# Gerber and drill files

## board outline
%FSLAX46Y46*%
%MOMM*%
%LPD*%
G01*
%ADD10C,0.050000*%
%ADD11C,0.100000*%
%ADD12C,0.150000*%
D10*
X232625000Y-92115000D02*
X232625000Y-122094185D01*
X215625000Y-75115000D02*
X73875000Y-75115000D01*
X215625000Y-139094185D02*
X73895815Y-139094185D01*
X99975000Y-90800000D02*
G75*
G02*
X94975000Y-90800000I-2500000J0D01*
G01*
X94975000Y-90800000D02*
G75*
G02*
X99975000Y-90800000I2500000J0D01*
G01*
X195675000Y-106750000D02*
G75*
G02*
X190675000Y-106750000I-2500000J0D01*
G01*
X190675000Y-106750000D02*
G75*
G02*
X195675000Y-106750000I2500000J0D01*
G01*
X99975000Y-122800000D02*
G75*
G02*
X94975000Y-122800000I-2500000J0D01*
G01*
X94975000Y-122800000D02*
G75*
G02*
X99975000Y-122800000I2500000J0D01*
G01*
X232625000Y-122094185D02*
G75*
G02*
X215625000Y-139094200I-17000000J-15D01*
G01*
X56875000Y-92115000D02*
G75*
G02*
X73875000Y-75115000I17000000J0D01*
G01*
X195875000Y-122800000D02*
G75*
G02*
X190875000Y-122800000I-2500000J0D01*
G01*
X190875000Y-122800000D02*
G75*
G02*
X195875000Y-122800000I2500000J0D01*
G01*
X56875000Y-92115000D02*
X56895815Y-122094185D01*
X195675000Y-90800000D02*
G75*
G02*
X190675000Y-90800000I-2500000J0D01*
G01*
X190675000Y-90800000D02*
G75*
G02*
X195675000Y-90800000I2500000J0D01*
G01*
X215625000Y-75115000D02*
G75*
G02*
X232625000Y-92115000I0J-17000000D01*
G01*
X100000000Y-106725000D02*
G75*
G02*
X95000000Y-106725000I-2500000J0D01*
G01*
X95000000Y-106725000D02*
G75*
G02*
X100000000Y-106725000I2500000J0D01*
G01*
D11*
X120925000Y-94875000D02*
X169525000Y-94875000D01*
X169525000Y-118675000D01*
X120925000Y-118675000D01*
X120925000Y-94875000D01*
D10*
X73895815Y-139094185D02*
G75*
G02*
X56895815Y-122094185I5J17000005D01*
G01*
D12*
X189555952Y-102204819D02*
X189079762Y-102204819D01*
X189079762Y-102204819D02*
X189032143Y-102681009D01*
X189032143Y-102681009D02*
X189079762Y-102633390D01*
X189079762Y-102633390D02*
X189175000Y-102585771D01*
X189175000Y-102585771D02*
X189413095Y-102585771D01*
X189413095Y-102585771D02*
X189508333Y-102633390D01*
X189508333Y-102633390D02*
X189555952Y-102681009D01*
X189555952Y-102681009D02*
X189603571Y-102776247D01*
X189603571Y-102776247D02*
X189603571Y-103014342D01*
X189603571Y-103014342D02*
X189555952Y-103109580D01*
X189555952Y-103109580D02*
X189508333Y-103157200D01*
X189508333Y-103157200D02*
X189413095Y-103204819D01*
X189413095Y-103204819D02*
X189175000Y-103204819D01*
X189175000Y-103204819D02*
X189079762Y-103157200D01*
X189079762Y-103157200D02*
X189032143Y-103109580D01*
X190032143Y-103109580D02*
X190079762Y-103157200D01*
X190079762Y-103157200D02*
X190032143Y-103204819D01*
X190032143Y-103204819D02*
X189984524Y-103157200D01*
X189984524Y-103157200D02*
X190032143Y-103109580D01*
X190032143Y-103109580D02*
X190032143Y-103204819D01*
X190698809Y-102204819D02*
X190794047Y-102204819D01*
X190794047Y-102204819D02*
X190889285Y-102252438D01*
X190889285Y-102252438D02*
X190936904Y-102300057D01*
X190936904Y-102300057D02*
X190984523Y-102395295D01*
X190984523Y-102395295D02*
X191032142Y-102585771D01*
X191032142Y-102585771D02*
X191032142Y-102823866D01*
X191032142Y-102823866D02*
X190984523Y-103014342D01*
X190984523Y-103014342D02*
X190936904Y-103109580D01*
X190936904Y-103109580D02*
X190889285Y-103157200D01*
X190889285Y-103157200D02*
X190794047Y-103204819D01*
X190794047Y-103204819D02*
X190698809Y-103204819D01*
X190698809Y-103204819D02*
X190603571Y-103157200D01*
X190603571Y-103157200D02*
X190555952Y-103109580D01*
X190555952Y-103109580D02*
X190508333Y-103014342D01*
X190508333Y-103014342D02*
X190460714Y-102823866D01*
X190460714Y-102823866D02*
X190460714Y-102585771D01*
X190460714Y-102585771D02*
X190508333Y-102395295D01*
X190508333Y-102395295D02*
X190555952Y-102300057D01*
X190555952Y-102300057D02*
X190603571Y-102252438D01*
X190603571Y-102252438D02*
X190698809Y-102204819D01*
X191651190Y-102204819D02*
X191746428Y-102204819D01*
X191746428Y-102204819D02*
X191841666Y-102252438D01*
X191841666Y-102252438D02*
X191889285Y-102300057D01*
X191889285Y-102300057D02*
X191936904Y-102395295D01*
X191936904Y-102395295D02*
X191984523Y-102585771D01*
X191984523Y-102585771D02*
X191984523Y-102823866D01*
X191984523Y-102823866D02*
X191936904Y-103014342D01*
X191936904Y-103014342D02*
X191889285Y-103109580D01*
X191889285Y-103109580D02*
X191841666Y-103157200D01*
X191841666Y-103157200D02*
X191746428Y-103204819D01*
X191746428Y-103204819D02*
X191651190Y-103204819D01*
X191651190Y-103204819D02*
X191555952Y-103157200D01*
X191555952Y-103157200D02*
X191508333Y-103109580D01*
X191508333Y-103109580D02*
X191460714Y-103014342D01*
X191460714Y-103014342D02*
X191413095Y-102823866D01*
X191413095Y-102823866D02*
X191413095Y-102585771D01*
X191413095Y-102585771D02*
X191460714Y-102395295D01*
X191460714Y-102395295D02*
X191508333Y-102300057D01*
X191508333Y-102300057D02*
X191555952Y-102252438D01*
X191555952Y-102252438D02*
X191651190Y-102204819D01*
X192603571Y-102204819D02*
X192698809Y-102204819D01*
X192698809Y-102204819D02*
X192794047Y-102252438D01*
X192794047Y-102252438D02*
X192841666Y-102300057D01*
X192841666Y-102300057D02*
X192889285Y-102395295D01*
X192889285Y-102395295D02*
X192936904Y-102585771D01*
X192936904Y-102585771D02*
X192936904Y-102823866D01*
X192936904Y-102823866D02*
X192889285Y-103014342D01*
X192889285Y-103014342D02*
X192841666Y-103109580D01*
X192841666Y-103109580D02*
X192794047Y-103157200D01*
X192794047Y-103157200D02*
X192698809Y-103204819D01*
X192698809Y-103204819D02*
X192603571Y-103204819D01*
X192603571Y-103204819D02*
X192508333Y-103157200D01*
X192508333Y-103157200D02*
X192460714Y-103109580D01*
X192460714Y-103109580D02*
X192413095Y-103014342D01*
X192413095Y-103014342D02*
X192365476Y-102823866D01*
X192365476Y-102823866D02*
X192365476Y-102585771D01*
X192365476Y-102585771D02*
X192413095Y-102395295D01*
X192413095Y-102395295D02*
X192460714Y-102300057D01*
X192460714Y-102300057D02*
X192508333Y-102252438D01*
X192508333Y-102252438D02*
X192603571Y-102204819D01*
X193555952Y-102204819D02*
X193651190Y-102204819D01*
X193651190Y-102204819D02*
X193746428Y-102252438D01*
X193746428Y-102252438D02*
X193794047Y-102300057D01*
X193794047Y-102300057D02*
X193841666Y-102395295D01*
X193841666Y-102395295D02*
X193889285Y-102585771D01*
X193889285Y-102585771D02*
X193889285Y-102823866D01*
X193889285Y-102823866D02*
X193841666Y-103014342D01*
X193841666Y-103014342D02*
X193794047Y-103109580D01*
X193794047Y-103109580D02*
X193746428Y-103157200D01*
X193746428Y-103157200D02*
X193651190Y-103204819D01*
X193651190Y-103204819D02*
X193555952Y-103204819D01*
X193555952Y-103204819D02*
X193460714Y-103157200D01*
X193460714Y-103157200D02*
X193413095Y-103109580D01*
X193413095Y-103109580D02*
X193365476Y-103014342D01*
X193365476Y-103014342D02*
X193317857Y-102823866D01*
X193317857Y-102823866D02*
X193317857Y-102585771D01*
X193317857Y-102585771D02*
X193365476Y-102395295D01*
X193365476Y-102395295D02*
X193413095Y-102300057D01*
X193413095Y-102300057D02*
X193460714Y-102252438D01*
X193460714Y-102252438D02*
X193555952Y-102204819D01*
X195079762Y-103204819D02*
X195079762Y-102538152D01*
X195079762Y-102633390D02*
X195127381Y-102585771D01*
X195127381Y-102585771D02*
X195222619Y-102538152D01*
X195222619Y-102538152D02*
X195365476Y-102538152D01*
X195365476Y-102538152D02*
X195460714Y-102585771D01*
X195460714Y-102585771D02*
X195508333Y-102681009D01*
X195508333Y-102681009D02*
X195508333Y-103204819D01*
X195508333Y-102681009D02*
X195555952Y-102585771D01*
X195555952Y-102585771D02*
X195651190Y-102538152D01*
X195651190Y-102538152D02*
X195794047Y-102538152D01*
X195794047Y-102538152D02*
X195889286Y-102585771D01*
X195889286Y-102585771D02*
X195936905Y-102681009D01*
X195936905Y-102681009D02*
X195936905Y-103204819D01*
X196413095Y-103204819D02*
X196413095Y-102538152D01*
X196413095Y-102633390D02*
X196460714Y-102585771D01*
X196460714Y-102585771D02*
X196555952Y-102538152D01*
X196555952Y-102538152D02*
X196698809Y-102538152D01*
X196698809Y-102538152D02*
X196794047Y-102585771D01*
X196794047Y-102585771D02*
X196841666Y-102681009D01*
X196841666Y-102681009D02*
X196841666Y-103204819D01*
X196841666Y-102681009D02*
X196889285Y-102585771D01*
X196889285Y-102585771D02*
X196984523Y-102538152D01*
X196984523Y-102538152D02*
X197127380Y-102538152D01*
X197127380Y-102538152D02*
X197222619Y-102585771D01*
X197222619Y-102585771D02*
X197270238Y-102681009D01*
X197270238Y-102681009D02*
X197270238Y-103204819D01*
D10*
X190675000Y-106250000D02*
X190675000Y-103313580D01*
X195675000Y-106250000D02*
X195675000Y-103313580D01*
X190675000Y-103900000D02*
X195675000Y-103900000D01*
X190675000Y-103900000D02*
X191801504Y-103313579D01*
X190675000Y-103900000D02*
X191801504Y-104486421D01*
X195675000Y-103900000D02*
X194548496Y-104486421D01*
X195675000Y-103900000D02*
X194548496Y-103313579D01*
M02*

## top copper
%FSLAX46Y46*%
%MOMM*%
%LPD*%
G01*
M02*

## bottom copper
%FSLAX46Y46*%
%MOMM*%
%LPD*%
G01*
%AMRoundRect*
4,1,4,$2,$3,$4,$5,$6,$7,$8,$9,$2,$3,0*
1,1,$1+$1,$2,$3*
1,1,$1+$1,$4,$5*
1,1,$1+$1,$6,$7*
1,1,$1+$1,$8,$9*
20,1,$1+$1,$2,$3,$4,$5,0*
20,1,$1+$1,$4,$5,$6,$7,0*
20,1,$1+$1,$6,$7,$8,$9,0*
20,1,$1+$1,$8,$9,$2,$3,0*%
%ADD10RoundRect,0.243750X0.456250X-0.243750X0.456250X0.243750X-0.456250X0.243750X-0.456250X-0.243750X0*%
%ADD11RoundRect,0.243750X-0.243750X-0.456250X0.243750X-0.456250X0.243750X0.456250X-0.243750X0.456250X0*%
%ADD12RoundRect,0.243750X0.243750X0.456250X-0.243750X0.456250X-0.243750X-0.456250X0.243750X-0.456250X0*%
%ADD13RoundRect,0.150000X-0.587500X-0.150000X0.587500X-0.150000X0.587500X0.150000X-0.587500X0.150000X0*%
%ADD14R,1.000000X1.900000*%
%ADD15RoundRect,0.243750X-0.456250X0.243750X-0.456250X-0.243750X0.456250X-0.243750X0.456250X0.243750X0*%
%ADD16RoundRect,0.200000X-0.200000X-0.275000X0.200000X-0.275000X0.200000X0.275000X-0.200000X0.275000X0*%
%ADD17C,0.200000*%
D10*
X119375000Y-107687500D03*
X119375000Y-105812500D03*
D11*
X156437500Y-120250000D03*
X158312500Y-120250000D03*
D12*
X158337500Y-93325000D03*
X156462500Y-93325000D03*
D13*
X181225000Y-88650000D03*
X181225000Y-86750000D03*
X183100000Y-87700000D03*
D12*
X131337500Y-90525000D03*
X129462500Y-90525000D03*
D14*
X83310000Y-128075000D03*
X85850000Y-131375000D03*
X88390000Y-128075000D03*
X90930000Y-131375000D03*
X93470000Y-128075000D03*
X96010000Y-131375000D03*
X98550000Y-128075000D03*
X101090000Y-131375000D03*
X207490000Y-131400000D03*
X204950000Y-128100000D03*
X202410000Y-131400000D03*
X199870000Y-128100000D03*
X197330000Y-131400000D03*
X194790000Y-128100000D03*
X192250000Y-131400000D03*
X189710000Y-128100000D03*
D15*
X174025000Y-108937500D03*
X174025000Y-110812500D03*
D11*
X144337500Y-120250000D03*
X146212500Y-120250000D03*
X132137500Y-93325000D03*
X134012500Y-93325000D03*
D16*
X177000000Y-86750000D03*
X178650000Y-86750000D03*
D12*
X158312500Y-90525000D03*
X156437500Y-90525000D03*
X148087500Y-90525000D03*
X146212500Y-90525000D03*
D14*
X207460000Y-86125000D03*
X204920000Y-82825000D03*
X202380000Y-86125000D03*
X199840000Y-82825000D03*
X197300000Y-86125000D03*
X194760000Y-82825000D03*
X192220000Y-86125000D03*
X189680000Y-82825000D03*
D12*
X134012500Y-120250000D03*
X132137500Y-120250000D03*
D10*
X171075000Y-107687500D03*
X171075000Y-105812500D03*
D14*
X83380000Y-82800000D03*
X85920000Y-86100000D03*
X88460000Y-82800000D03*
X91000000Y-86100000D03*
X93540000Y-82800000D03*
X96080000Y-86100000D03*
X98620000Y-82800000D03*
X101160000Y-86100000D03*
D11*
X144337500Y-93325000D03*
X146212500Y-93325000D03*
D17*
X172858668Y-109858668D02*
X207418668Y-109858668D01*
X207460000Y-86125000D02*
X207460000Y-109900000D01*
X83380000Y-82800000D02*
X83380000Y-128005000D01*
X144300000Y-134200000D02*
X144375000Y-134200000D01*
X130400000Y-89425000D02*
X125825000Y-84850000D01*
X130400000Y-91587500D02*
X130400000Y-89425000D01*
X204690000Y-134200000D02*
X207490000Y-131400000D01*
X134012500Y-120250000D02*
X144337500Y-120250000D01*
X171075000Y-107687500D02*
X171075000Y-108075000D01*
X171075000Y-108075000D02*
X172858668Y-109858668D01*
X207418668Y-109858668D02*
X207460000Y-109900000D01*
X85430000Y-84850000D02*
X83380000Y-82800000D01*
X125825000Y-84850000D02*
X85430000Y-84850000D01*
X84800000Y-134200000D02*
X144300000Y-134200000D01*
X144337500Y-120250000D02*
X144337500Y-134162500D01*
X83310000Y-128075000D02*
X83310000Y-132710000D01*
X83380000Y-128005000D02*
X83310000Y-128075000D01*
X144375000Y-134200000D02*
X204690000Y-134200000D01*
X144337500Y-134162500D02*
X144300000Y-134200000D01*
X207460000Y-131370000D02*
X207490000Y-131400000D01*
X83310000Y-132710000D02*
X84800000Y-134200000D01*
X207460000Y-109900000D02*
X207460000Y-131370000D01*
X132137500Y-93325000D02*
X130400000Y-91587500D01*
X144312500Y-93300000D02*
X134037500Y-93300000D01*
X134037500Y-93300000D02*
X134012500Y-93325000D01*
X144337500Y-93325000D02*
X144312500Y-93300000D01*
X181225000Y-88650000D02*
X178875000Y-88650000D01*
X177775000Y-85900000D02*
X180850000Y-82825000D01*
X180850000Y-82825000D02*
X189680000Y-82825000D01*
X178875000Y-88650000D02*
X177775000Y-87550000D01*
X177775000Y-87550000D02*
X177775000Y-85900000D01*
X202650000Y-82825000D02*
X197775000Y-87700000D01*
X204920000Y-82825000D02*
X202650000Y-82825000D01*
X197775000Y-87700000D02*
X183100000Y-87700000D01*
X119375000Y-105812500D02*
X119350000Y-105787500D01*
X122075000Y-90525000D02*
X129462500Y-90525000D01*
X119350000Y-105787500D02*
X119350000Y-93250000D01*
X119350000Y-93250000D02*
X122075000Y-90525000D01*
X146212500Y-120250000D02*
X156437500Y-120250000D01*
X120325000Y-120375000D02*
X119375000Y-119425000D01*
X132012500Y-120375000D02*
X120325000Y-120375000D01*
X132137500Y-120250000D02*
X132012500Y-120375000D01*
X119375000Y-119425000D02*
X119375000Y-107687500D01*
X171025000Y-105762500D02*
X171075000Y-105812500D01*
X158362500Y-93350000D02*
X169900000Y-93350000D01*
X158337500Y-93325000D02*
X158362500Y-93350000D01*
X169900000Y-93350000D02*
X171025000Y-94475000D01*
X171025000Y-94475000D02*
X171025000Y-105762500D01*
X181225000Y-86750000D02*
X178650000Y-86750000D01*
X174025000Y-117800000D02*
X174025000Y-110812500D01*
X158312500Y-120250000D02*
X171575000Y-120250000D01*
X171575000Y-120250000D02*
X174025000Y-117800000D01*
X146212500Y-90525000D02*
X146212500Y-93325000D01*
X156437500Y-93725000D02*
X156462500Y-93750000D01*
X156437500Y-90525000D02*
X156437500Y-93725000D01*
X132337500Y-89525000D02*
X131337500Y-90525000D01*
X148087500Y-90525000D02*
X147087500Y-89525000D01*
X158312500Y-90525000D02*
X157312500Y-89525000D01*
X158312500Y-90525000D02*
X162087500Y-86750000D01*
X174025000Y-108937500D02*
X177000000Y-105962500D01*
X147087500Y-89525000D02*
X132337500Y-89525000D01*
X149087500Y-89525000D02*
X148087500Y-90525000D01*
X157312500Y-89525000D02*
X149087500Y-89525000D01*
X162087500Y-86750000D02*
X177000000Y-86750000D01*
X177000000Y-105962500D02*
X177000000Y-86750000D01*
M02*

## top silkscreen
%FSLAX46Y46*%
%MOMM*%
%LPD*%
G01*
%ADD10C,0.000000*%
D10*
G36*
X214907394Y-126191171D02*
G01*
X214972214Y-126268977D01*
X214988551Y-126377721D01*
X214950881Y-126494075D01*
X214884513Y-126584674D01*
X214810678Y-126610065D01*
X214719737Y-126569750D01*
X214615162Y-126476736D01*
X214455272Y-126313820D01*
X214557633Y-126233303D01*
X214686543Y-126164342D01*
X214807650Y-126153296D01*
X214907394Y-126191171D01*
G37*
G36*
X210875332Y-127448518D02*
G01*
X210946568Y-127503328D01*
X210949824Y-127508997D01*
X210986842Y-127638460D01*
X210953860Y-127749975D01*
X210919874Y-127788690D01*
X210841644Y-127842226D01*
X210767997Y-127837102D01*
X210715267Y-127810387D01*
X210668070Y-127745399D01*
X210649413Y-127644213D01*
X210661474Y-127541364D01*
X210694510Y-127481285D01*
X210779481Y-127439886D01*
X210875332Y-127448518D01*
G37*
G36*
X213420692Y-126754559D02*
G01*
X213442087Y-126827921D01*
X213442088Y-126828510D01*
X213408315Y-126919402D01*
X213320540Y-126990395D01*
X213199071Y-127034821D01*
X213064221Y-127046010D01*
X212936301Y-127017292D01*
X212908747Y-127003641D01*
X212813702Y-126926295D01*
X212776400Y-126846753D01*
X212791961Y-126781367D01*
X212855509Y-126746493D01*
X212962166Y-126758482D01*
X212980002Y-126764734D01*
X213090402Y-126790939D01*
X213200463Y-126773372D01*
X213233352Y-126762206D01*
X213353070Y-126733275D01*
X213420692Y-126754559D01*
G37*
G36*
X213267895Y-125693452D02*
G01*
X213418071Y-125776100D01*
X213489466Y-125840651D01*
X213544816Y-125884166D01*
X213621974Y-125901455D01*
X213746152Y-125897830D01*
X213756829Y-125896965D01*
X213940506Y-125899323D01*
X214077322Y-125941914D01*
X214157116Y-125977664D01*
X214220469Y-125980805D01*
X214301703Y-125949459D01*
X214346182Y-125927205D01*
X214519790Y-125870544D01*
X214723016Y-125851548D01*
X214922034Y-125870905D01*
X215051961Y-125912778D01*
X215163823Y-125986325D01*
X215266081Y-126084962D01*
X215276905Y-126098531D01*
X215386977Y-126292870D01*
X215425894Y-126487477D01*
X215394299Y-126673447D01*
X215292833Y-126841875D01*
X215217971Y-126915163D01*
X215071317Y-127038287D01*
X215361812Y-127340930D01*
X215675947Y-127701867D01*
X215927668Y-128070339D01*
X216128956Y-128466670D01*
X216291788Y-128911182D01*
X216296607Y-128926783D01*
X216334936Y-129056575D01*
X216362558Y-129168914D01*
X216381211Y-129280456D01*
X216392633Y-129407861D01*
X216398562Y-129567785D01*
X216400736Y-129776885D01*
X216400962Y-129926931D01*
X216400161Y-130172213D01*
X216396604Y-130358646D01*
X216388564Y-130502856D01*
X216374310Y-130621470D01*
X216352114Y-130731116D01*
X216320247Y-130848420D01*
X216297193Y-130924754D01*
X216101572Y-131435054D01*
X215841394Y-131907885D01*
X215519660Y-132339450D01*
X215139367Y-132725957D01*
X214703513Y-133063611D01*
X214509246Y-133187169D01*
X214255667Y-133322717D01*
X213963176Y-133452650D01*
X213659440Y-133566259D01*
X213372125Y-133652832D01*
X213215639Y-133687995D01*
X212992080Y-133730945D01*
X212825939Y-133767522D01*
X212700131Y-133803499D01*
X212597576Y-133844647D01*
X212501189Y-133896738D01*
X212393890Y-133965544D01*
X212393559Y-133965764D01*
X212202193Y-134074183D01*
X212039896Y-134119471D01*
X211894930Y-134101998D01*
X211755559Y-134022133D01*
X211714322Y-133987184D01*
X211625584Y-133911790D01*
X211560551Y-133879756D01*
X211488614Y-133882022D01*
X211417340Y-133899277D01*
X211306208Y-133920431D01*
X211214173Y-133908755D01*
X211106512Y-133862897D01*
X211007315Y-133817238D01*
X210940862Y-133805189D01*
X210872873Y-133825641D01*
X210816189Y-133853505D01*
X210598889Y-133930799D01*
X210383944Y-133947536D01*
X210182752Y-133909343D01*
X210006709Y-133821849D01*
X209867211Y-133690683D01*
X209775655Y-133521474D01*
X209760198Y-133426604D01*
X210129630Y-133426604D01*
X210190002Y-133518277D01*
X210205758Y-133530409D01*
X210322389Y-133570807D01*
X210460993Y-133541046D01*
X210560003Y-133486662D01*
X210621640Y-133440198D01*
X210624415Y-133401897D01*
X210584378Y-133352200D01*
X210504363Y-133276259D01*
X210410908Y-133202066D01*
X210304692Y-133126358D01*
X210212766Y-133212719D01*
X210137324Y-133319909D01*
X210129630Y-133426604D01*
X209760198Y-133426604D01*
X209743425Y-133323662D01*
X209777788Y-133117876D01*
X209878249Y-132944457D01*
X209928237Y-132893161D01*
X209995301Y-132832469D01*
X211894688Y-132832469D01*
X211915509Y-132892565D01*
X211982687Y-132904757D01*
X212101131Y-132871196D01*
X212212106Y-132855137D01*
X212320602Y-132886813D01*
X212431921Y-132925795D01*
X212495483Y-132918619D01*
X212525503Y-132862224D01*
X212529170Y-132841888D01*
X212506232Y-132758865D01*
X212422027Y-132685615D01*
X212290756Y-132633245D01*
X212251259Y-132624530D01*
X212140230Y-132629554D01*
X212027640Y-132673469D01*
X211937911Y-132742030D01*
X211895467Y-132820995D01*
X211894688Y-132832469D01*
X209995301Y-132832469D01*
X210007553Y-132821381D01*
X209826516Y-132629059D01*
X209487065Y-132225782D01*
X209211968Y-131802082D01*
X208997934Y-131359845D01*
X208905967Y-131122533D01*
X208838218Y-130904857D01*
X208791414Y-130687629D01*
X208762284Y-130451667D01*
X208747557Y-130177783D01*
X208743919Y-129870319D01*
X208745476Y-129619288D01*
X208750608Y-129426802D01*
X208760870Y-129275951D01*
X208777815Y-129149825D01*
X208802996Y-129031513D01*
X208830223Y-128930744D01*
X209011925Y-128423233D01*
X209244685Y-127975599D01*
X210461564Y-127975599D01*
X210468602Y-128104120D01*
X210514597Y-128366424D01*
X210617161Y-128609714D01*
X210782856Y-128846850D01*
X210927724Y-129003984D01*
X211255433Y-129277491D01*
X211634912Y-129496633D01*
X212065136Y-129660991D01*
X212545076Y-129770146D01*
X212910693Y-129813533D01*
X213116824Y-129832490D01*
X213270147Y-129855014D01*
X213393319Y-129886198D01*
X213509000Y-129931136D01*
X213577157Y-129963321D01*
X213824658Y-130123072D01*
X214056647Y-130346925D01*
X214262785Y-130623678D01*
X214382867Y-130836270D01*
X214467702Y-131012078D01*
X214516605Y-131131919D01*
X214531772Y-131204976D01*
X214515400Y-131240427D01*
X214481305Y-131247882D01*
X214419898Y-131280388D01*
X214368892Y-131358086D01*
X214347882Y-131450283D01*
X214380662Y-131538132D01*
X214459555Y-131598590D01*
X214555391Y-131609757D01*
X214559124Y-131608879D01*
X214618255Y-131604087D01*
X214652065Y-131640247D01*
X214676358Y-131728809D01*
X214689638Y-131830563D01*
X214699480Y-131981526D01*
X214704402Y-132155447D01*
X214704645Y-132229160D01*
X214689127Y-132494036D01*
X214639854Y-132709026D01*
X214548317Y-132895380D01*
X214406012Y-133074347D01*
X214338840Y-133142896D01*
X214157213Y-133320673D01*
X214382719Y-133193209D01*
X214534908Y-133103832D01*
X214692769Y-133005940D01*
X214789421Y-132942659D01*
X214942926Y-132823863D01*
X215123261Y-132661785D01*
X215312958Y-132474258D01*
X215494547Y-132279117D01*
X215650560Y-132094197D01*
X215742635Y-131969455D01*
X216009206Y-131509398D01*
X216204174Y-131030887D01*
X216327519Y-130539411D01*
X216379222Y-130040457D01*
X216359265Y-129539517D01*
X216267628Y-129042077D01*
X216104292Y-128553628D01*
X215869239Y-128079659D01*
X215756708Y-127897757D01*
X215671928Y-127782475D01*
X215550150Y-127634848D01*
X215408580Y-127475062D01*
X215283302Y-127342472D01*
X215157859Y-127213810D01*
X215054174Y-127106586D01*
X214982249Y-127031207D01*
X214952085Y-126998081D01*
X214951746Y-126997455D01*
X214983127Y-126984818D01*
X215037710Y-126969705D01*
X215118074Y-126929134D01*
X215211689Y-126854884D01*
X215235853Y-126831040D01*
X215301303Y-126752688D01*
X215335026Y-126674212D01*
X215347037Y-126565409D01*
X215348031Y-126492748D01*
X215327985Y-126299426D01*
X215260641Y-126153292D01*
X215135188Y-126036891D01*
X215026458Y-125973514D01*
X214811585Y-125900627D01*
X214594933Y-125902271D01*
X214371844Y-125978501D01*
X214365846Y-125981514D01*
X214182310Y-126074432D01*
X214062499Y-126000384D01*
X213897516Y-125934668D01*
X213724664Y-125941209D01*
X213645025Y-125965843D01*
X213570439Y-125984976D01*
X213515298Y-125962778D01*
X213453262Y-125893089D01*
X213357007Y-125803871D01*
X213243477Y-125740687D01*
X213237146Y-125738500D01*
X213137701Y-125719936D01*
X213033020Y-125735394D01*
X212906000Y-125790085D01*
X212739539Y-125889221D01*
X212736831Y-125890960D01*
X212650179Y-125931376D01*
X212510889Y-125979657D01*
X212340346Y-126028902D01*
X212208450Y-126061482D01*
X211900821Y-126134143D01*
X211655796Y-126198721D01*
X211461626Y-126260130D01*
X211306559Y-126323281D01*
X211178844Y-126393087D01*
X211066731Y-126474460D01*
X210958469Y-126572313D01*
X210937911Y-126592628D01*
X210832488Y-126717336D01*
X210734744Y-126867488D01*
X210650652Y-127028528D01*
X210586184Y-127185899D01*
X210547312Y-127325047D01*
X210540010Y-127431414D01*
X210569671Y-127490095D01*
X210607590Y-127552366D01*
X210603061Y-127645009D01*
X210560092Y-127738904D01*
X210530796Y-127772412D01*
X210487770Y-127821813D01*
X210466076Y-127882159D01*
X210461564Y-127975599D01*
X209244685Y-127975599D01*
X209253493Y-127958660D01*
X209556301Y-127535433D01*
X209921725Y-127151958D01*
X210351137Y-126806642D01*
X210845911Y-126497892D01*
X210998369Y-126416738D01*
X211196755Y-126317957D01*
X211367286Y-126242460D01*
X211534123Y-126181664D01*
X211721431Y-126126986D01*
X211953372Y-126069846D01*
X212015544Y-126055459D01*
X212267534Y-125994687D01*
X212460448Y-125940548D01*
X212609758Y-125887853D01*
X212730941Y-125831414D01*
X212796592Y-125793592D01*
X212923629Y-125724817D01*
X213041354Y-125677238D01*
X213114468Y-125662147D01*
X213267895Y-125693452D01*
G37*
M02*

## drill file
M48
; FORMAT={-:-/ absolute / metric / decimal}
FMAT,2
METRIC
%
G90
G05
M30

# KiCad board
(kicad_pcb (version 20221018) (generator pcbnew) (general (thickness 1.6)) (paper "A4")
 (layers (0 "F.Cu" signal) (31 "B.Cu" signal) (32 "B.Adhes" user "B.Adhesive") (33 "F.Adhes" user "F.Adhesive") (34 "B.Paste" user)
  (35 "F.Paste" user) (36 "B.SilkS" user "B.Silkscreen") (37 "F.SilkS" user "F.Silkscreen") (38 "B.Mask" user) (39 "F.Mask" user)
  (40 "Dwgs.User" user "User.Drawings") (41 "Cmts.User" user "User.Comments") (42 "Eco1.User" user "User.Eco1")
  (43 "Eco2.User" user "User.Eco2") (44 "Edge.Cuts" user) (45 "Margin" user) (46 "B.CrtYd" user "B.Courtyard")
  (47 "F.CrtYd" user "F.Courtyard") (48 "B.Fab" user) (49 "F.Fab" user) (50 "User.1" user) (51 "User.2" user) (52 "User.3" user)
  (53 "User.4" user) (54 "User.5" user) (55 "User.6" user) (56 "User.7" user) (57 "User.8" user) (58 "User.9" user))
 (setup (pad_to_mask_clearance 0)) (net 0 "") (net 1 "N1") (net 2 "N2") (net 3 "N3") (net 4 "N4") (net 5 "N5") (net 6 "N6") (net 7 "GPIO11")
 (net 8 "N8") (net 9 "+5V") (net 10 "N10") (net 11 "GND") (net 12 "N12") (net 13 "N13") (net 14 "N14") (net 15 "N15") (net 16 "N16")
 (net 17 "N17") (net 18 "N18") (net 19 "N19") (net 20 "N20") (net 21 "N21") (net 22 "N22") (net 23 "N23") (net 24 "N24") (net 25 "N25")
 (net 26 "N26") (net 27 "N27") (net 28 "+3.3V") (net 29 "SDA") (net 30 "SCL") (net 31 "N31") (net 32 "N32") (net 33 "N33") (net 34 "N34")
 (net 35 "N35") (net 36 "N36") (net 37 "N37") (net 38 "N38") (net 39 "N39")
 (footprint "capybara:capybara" (layer "F.Cu") (at 212.725 129.625)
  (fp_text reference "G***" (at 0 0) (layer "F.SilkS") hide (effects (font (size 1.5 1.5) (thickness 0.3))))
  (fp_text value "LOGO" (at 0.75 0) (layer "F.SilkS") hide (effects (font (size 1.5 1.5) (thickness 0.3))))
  (fp_poly
   (pts (xy 2.182394 -3.433829) (xy 2.247214 -3.356023) (xy 2.263551 -3.247279) (xy 2.225881 -3.130925) (xy 2.159513 -3.040326)
    (xy 2.085678 -3.014935) (xy 1.994737 -3.05525) (xy 1.890162 -3.148264) (xy 1.730272 -3.31118) (xy 1.832633 -3.391697)
    (xy 1.961543 -3.460658) (xy 2.08265 -3.471704))
   (stroke (width 0) (type solid)) (fill solid) (layer "F.SilkS"))
  (fp_poly
   (pts (xy -1.849668 -2.176482) (xy -1.778432 -2.121672) (xy -1.775176 -2.116003) (xy -1.738158 -1.98654) (xy -1.77114 -1.875025)
    (xy -1.805126 -1.83631) (xy -1.883356 -1.782774) (xy -1.957003 -1.787898) (xy -2.009733 -1.814613) (xy -2.05693 -1.879601)
    (xy -2.075587 -1.980787) (xy -2.063526 -2.083636) (xy -2.03049 -2.143715) (xy -1.945519 -2.185114))
   (stroke (width 0) (type solid)) (fill solid) (layer "F.SilkS"))
  (fp_poly
   (pts (xy 0.695692 -2.870441) (xy 0.717087 -2.797079) (xy 0.717088 -2.79649) (xy 0.683315 -2.705598) (xy 0.59554 -2.634605)
    (xy 0.474071 -2.590179) (xy 0.339221 -2.57899) (xy 0.211301 -2.607708) (xy 0.183747 -2.621359) (xy 0.088702 -2.698705)
    (xy 0.0514 -2.778247) (xy 0.066961 -2.843633) (xy 0.130509 -2.878507) (xy 0.237166 -2.866518) (xy 0.255002 -2.860266)
    (xy 0.365402 -2.834061) (xy 0.475463 -2.851628) (xy 0.508352 -2.862794) (xy 0.62807 -2.891725))
   (stroke (width 0) (type solid)) (fill solid) (layer "F.SilkS"))
  (fp_poly
   (pts (xy 0.542895 -3.931548) (xy 0.693071 -3.8489) (xy 0.764466 -3.784349) (xy 0.819816 -3.740834) (xy 0.896974 -3.723545)
    (xy 1.021152 -3.72717) (xy 1.031829 -3.728035) (xy 1.215506 -3.725677) (xy 1.352322 -3.683086) (xy 1.432116 -3.647336)
    (xy 1.495469 -3.644195) (xy 1.576703 -3.675541) (xy 1.621182 -3.697795) (xy 1.79479 -3.754456) (xy 1.998016 -3.773452)
    (xy 2.197034 -3.754095) (xy 2.326961 -3.712222) (xy 2.438823 -3.638675) (xy 2.541081 -3.540038) (xy 2.551905 -3.526469)
    (xy 2.661977 -3.33213) (xy 2.700894 -3.137523) (xy 2.669299 -2.951553) (xy 2.567833 -2.783125) (xy 2.492971 -2.709837)
    (xy 2.346317 -2.586713) (xy 2.636812 -2.28407) (xy 2.950947 -1.923133) (xy 3.202668 -1.554661) (xy 3.403956 -1.15833)
    (xy 3.566788 -0.713818) (xy 3.571607 -0.698217) (xy 3.609936 -0.568425) (xy 3.637558 -0.456086) (xy 3.656211 -0.344544)
    (xy 3.667633 -0.217139) (xy 3.673562 -0.057215) (xy 3.675736 0.151885) (xy 3.675962 0.301931) (xy 3.675161 0.547213)
    (xy 3.671604 0.733646) (xy 3.663564 0.877856) (xy 3.64931 0.99647) (xy 3.627114 1.106116) (xy 3.595247 1.22342) (xy 3.572193 1.299754)
    (xy 3.376572 1.810054) (xy 3.116394 2.282885) (xy 2.79466 2.71445) (xy 2.414367 3.100957) (xy 1.978513 3.438611) (xy 1.784246 3.562169)
    (xy 1.530667 3.697717) (xy 1.238176 3.82765) (xy 0.93444 3.941259) (xy 0.647125 4.027832) (xy 0.490639 4.062995) (xy 0.26708 4.105945)
    (xy 0.100939 4.142522) (xy -0.024869 4.178499) (xy -0.127424 4.219647) (xy -0.223811 4.271738) (xy -0.33111 4.340544)
    (xy -0.331441 4.340764) (xy -0.522807 4.449183) (xy -0.685104 4.494471) (xy -0.83007 4.476998) (xy -0.969441 4.397133)
    (xy -1.010678 4.362184) (xy -1.099416 4.28679) (xy -1.164449 4.254756) (xy -1.236386 4.257022) (xy -1.30766 4.274277)
    (xy -1.418792 4.295431) (xy -1.510827 4.283755) (xy -1.618488 4.237897) (xy -1.717685 4.192238) (xy -1.784138 4.180189)
    (xy -1.852127 4.200641) (xy -1.908811 4.228505) (xy -2.126111 4.305799) (xy -2.341056 4.322536) (xy -2.542248 4.284343)
    (xy -2.718291 4.196849) (xy -2.857789 4.065683) (xy -2.949345 3.896474) (xy -2.964802 3.801604) (xy -2.59537 3.801604)
    (xy -2.534998 3.893277) (xy -2.519242 3.905409) (xy -2.402611 3.945807) (xy -2.264007 3.916046) (xy -2.164997 3.861662)
    (xy -2.10336 3.815198) (xy -2.100585 3.776897) (xy -2.140622 3.7272) (xy -2.220637 3.651259) (xy -2.314092 3.577066)
    (xy -2.420308 3.501358) (xy -2.512234 3.587719) (xy -2.587676 3.694909) (xy -2.59537 3.801604) (xy -2.964802 3.801604)
    (xy -2.981575 3.698662) (xy -2.947212 3.492876) (xy -2.846751 3.319457) (xy -2.796763 3.268161) (xy -2.729699 3.207469)
    (xy -0.830312 3.207469) (xy -0.809491 3.267565) (xy -0.742313 3.279757) (xy -0.623869 3.246196) (xy -0.512894 3.230137)
    (xy -0.404398 3.261813) (xy -0.293079 3.300795) (xy -0.229517 3.293619) (xy -0.199497 3.237224) (xy -0.19583 3.216888)
    (xy -0.218768 3.133865) (xy -0.302973 3.060615) (xy -0.434244 3.008245) (xy -0.473741 2.99953) (xy -0.58477 3.004554)
    (xy -0.69736 3.048469) (xy -0.787089 3.11703) (xy -0.829533 3.195995) (xy -0.830312 3.207469) (xy -2.729699 3.207469)
    (xy -2.717447 3.196381) (xy -2.898484 3.004059) (xy -3.237935 2.600782) (xy -3.513032 2.177082) (xy -3.727066 1.734845)
    (xy -3.819033 1.497533) (xy -3.886782 1.279857) (xy -3.933586 1.062629) (xy -3.962716 0.826667) (xy -3.977443 0.552783)
    (xy -3.981081 0.245319) (xy -3.979524 -0.005712) (xy -3.974392 -0.198198) (xy -3.96413 -0.349049) (xy -3.947185 -0.475175)
    (xy -3.922004 -0.593487) (xy -3.894777 -0.694256) (xy -3.713075 -1.201767) (xy -3.480315 -1.649401) (xy -2.263436 -1.649401)
    (xy -2.256398 -1.52088) (xy -2.210403 -1.258576) (xy -2.107839 -1.015286) (xy -1.942144 -0.77815) (xy -1.797276 -0.621016)
    (xy -1.469567 -0.347509) (xy -1.090088 -0.128367) (xy -0.659864 0.035991) (xy -0.179924 0.145146) (xy 0.185693 0.188533)
    (xy 0.391824 0.20749) (xy 0.545147 0.230014) (xy 0.668319 0.261198) (xy 0.784 0.306136) (xy 0.852157 0.338321) (xy 1.099658 0.498072)
    (xy 1.331647 0.721925) (xy 1.537785 0.998678) (xy 1.657867 1.21127) (xy 1.742702 1.387078) (xy 1.791605 1.506919) (xy 1.806772 1.579976)
    (xy 1.7904 1.615427) (xy 1.756305 1.622882) (xy 1.694898 1.655388) (xy 1.643892 1.733086) (xy 1.622882 1.825283) (xy 1.655662 1.913132)
    (xy 1.734555 1.97359) (xy 1.830391 1.984757) (xy 1.834124 1.983879) (xy 1.893255 1.979087) (xy 1.927065 2.015247) (xy 1.951358 2.103809)
    (xy 1.964638 2.205563) (xy 1.97448 2.356526) (xy 1.979402 2.530447) (xy 1.979645 2.60416) (xy 1.964127 2.869036) (xy 1.914854 3.084026)
    (xy 1.823317 3.27038) (xy 1.681012 3.449347) (xy 1.61384 3.517896) (xy 1.432213 3.695673) (xy 1.657719 3.568209) (xy 1.809908 3.478832)
    (xy 1.967769 3.38094) (xy 2.064421 3.317659) (xy 2.217926 3.198863) (xy 2.398261 3.036785) (xy 2.587958 2.849258) (xy 2.769547 2.654117)
    (xy 2.92556 2.469197) (xy 3.017635 2.344455) (xy 3.284206 1.884398) (xy 3.479174 1.405887) (xy 3.602519 0.914411) (xy 3.654222 0.415457)
    (xy 3.634265 -0.085483) (xy 3.542628 -0.582923) (xy 3.379292 -1.071372) (xy 3.144239 -1.545341) (xy 3.031708 -1.727243)
    (xy 2.946928 -1.842525) (xy 2.82515 -1.990152) (xy 2.68358 -2.149938) (xy 2.558302 -2.282528) (xy 2.432859 -2.41119)
    (xy 2.329174 -2.518414) (xy 2.257249 -2.593793) (xy 2.227085 -2.626919) (xy 2.226746 -2.627545) (xy 2.258127 -2.640182)
    (xy 2.31271 -2.655295) (xy 2.393074 -2.695866) (xy 2.486689 -2.770116) (xy 2.510853 -2.79396) (xy 2.576303 -2.872312)
    (xy 2.610026 -2.950788) (xy 2.622037 -3.059591) (xy 2.623031 -3.132252) (xy 2.602985 -3.325574) (xy 2.535641 -3.471708)
    (xy 2.410188 -3.588109) (xy 2.301458 -3.651486) (xy 2.086585 -3.724373) (xy 1.869933 -3.722729) (xy 1.646844 -3.646499)
    (xy 1.640846 -3.643486) (xy 1.45731 -3.550568) (xy 1.337499 -3.624616) (xy 1.172516 -3.690332) (xy 0.999664 -3.683791)
    (xy 0.920025 -3.659157) (xy 0.845439 -3.640024) (xy 0.790298 -3.662222) (xy 0.728262 -3.731911) (xy 0.632007 -3.821129)
    (xy 0.518477 -3.884313) (xy 0.512146 -3.8865) (xy 0.412701 -3.905064) (xy 0.30802 -3.889606) (xy 0.181 -3.834915)
    (xy 0.014539 -3.735779) (xy 0.011831 -3.73404) (xy -0.074821 -3.693624) (xy -0.214111 -3.645343) (xy -0.384654 -3.596098)
    (xy -0.51655 -3.563518) (xy -0.824179 -3.490857) (xy -1.069204 -3.426279) (xy -1.263374 -3.36487) (xy -1.418441 -3.301719)
    (xy -1.546156 -3.231913) (xy -1.658269 -3.15054) (xy -1.766531 -3.052687) (xy -1.787089 -3.032372) (xy -1.892512 -2.907664)
    (xy -1.990256 -2.757512) (xy -2.074348 -2.596472) (xy -2.138816 -2.439101) (xy -2.177688 -2.299953) (xy -2.18499 -2.193586)
    (xy -2.155329 -2.134905) (xy -2.11741 -2.072634) (xy -2.121939 -1.979991) (xy -2.164908 -1.886096) (xy -2.194204 -1.852588)
    (xy -2.23723 -1.803187) (xy -2.258924 -1.742841) (xy -2.263436 -1.649401) (xy -3.480315 -1.649401) (xy -3.471507 -1.66634)
    (xy -3.168699 -2.089567) (xy -2.803275 -2.473042) (xy -2.373863 -2.818358) (xy -1.879089 -3.127108) (xy -1.726631 -3.208262)
    (xy -1.528245 -3.307043) (xy -1.357714 -3.38254) (xy -1.190877 -3.443336) (xy -1.003569 -3.498014) (xy -0.771628 -3.555154)
    (xy -0.709456 -3.569541) (xy -0.457466 -3.630313) (xy -0.264552 -3.684452) (xy -0.115242 -3.737147) (xy 0.005941 -3.793586)
    (xy 0.071592 -3.831408) (xy 0.198629 -3.900183) (xy 0.316354 -3.947762) (xy 0.389468 -3.962853))
   (stroke (width 0) (type solid)) (fill solid) (layer "F.SilkS")))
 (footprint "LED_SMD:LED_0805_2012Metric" (layer "B.Cu") (at 119.375 106.75 90)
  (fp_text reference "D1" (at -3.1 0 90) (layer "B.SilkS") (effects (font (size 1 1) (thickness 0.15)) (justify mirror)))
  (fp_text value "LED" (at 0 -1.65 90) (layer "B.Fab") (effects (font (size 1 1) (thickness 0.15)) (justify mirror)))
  (pad "1" smd roundrect (at -0.9375 0 90) (size 0.975 1.4) (layers "B.Cu" "B.Paste" "B.Mask") (roundrect_rratio 0.25) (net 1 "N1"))
  (pad "2" smd roundrect (at 0.9375 0 90) (size 0.975 1.4) (layers "B.Cu" "B.Paste" "B.Mask") (roundrect_rratio 0.25) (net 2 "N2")))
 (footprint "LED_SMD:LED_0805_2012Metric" (layer "B.Cu") (at 157.375 120.25)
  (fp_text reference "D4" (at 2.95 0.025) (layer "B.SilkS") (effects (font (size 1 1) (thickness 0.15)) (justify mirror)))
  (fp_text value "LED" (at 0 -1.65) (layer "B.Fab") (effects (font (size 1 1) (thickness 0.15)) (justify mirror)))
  (pad "1" smd roundrect (at -0.9375 0) (size 0.975 1.4) (layers "B.Cu" "B.Paste" "B.Mask") (roundrect_rratio 0.25) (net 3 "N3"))
  (pad "2" smd roundrect (at 0.9375 0) (size 0.975 1.4) (layers "B.Cu" "B.Paste" "B.Mask") (roundrect_rratio 0.25) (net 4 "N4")))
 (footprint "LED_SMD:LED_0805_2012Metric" (layer "B.Cu") (at 157.4 93.325 180)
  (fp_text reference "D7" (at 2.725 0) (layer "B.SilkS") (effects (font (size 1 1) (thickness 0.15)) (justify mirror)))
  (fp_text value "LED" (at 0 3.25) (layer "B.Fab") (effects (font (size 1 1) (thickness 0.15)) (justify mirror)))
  (pad "1" smd roundrect (at -0.9375 0 180) (size 0.975 1.4) (layers "B.Cu" "B.Paste" "B.Mask") (roundrect_rratio 0.25) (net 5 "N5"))
  (pad "2" smd roundrect (at 0.9375 0 180) (size 0.975 1.4) (layers "B.Cu" "B.Paste" "B.Mask") (roundrect_rratio 0.25) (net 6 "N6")))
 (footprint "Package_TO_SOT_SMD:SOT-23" (layer "B.Cu") (at 182.1625 87.7)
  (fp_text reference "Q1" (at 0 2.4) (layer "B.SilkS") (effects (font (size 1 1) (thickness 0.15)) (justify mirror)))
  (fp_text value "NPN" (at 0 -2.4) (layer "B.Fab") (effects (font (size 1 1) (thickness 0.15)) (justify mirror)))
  (pad "1" smd roundrect (at -0.9375 0.95) (size 1.475 0.6) (layers "B.Cu" "B.Paste" "B.Mask") (roundrect_rratio 0.25) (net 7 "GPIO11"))
  (pad "2" smd roundrect (at -0.9375 -0.95) (size 1.475 0.6) (layers "B.Cu" "B.Paste" "B.Mask") (roundrect_rratio 0.25) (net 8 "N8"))
  (pad "3" smd roundrect (at 0.9375 0) (size 1.475 0.6) (layers "B.Cu" "B.Paste" "B.Mask") (roundrect_rratio 0.25) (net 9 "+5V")))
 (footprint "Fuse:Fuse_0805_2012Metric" (layer "B.Cu") (at 130.4 90.525 180)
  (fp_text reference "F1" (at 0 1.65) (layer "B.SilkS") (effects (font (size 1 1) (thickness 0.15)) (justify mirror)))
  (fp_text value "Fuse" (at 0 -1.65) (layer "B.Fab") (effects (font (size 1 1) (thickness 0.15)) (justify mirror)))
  (pad "1" smd roundrect (at -0.9375 0 180) (size 0.975 1.4) (layers "B.Cu" "B.Paste" "B.Mask") (roundrect_rratio 0.25) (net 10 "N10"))
  (pad "2" smd roundrect (at 0.9375 0 180) (size 0.975 1.4) (layers "B.Cu" "B.Paste" "B.Mask") (roundrect_rratio 0.25) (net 2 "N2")))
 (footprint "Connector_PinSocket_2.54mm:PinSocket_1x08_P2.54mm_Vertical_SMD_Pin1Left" (layer "B.Cu") (at 92.2 129.725 -90)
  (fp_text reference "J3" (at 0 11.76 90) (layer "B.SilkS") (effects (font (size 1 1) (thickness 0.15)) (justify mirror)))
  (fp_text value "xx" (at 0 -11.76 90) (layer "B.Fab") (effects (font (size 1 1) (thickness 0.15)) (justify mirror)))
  (pad "1" smd rect (at -1.65 8.89 270) (size 1.9 1) (layers "B.Cu" "B.Paste" "B.Mask") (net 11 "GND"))
  (pad "2" smd rect (at 1.65 6.35 270) (size 1.9 1) (layers "B.Cu" "B.Paste" "B.Mask") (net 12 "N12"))
  (pad "3" smd rect (at -1.65 3.81 270) (size 1.9 1) (layers "B.Cu" "B.Paste" "B.Mask") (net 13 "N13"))
  (pad "4" smd rect (at 1.65 1.27 270) (size 1.9 1) (layers "B.Cu" "B.Paste" "B.Mask") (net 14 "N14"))
  (pad "5" smd rect (at -1.65 -1.27 270) (size 1.9 1) (layers "B.Cu" "B.Paste" "B.Mask") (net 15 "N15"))
  (pad "6" smd rect (at 1.65 -3.81 270) (size 1.9 1) (layers "B.Cu" "B.Paste" "B.Mask") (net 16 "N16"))
  (pad "7" smd rect (at -1.65 -6.35 270) (size 1.9 1) (layers "B.Cu" "B.Paste" "B.Mask") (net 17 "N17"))
  (pad "8" smd rect (at 1.65 -8.89 270) (size 1.9 1) (layers "B.Cu" "B.Paste" "B.Mask") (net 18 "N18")))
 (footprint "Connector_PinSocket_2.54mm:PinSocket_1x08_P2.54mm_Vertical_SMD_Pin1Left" (layer "B.Cu") (at 198.6 129.75 90)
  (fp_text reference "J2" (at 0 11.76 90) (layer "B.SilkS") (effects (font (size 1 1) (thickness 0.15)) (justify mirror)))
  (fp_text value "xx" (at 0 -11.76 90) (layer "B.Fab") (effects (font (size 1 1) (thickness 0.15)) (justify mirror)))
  (pad "1" smd rect (at -1.65 8.89 90) (size 1.9 1) (layers "B.Cu" "B.Paste" "B.Mask") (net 11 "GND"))
  (pad "2" smd rect (at 1.65 6.35 90) (size 1.9 1) (layers "B.Cu" "B.Paste" "B.Mask") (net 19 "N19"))
  (pad "3" smd rect (at -1.65 3.81 90) (size 1.9 1) (layers "B.Cu" "B.Paste" "B.Mask") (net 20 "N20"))
  (pad "4" smd rect (at 1.65 1.27 90) (size 1.9 1) (layers "B.Cu" "B.Paste" "B.Mask") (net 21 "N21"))
  (pad "5" smd rect (at -1.65 -1.27 90) (size 1.9 1) (layers "B.Cu" "B.Paste" "B.Mask") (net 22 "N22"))
  (pad "6" smd rect (at 1.65 -3.81 90) (size 1.9 1) (layers "B.Cu" "B.Paste" "B.Mask") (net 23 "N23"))
  (pad "7" smd rect (at -1.65 -6.35 90) (size 1.9 1) (layers "B.Cu" "B.Paste" "B.Mask") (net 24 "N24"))
  (pad "8" smd rect (at 1.65 -8.89 90) (size 1.9 1) (layers "B.Cu" "B.Paste" "B.Mask") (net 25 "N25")))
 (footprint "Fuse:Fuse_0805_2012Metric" (layer "B.Cu") (at 174.025 109.875 -90)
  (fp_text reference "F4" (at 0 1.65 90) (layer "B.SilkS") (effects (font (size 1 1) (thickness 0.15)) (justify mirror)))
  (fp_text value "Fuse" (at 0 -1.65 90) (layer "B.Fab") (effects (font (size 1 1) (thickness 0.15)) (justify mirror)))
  (pad "1" smd roundrect (at -0.9375 0 270) (size 0.975 1.4) (layers "B.Cu" "B.Paste" "B.Mask") (roundrect_rratio 0.25) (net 10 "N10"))
  (pad "2" smd roundrect (at 0.9375 0 270) (size 0.975 1.4) (layers "B.Cu" "B.Paste" "B.Mask") (roundrect_rratio 0.25) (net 4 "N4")))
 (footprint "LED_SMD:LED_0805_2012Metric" (layer "B.Cu") (at 145.275 120.25)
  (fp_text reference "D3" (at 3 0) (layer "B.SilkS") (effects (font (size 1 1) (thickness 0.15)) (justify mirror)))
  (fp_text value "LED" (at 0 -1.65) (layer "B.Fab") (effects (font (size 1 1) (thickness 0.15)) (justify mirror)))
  (pad "1" smd roundrect (at -0.9375 0) (size 0.975 1.4) (layers "B.Cu" "B.Paste" "B.Mask") (roundrect_rratio 0.25) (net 11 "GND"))
  (pad "2" smd roundrect (at 0.9375 0) (size 0.975 1.4) (layers "B.Cu" "B.Paste" "B.Mask") (roundrect_rratio 0.25) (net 3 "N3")))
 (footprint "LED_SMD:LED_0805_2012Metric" (layer "B.Cu") (at 133.075 93.325)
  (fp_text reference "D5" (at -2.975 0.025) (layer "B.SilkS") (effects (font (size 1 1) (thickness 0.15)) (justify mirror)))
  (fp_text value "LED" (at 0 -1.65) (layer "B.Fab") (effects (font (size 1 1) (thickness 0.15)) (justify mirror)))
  (pad "1" smd roundrect (at -0.9375 0) (size 0.975 1.4) (layers "B.Cu" "B.Paste" "B.Mask") (roundrect_rratio 0.25) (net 11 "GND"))
  (pad "2" smd roundrect (at 0.9375 0) (size 0.975 1.4) (layers "B.Cu" "B.Paste" "B.Mask") (roundrect_rratio 0.25) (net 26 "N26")))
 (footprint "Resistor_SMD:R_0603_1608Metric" (layer "B.Cu") (at 177.825 86.75)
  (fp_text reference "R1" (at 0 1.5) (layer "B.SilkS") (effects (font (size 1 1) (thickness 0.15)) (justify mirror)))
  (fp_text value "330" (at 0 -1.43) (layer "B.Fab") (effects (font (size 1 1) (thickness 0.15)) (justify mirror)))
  (pad "1" smd roundrect (at -0.825 0) (size 0.8 0.95) (layers "B.Cu" "B.Paste" "B.Mask") (roundrect_rratio 0.25) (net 10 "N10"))
  (pad "2" smd roundrect (at 0.825 0) (size 0.8 0.95) (layers "B.Cu" "B.Paste" "B.Mask") (roundrect_rratio 0.25) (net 8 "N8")))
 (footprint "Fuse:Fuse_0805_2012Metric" (layer "B.Cu") (at 157.375 90.525 180)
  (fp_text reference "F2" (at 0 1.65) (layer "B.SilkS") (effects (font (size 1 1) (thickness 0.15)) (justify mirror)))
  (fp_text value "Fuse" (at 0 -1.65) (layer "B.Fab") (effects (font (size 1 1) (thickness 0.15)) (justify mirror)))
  (pad "1" smd roundrect (at -0.9375 0 180) (size 0.975 1.4) (layers "B.Cu" "B.Paste" "B.Mask") (roundrect_rratio 0.25) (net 10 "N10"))
  (pad "2" smd roundrect (at 0.9375 0 180) (size 0.975 1.4) (layers "B.Cu" "B.Paste" "B.Mask") (roundrect_rratio 0.25) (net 6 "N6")))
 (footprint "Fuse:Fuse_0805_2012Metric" (layer "B.Cu") (at 147.15 90.525 180)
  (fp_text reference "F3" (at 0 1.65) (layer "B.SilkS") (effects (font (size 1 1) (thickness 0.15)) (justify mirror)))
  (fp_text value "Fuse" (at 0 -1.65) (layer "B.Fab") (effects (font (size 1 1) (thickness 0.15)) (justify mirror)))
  (pad "1" smd roundrect (at -0.9375 0 180) (size 0.975 1.4) (layers "B.Cu" "B.Paste" "B.Mask") (roundrect_rratio 0.25) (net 10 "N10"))
  (pad "2" smd roundrect (at 0.9375 0 180) (size 0.975 1.4) (layers "B.Cu" "B.Paste" "B.Mask") (roundrect_rratio 0.25) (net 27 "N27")))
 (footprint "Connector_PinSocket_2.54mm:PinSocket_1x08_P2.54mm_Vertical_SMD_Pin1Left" (layer "B.Cu") (at 198.57 84.475 90)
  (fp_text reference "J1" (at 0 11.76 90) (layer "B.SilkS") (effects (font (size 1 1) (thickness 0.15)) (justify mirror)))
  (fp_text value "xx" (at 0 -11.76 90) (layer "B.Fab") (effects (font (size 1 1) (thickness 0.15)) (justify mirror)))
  (pad "1" smd rect (at -1.65 8.89 90) (size 1.9 1) (layers "B.Cu" "B.Paste" "B.Mask") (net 11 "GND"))
  (pad "2" smd rect (at 1.65 6.35 90) (size 1.9 1) (layers "B.Cu" "B.Paste" "B.Mask") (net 9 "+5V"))
  (pad "3" smd rect (at -1.65 3.81 90) (size 1.9 1) (layers "B.Cu" "B.Paste" "B.Mask") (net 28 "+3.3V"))
  (pad "4" smd rect (at 1.65 1.27 90) (size 1.9 1) (layers "B.Cu" "B.Paste" "B.Mask") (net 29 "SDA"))
  (pad "5" smd rect (at -1.65 -1.27 90) (size 1.9 1) (layers "B.Cu" "B.Paste" "B.Mask") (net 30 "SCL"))
  (pad "6" smd rect (at 1.65 -3.81 90) (size 1.9 1) (layers "B.Cu" "B.Paste" "B.Mask") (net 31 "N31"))
  (pad "7" smd rect (at -1.65 -6.35 90) (size 1.9 1) (layers "B.Cu" "B.Paste" "B.Mask") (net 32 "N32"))
  (pad "8" smd rect (at 1.65 -8.89 90) (size 1.9 1) (layers "B.Cu" "B.Paste" "B.Mask") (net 7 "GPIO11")))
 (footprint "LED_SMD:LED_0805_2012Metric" (layer "B.Cu") (at 133.075 120.25 180)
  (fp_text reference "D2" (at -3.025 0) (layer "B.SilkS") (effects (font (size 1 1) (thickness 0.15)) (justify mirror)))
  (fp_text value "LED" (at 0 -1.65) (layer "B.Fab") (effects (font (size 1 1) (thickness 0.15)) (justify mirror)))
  (pad "1" smd roundrect (at -0.9375 0 180) (size 0.975 1.4) (layers "B.Cu" "B.Paste" "B.Mask") (roundrect_rratio 0.25) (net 11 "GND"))
  (pad "2" smd roundrect (at 0.9375 0 180) (size 0.975 1.4) (layers "B.Cu" "B.Paste" "B.Mask") (roundrect_rratio 0.25) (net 1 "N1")))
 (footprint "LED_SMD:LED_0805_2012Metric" (layer "B.Cu") (at 171.075 106.75 90)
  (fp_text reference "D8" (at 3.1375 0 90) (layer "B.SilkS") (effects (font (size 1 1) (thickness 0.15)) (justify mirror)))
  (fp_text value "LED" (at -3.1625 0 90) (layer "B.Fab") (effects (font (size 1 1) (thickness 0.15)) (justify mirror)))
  (pad "1" smd roundrect (at -0.9375 0 90) (size 0.975 1.4) (layers "B.Cu" "B.Paste" "B.Mask") (roundrect_rratio 0.25) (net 11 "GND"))
  (pad "2" smd roundrect (at 0.9375 0 90) (size 0.975 1.4) (layers "B.Cu" "B.Paste" "B.Mask") (roundrect_rratio 0.25) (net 5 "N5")))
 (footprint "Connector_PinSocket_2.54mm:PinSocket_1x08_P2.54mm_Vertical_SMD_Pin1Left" (layer "B.Cu") (at 92.27 84.45 -90)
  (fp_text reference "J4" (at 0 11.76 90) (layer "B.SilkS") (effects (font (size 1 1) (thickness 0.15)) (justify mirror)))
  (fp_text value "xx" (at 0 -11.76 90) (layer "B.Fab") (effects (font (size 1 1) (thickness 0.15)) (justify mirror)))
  (pad "1" smd rect (at -1.65 8.89 270) (size 1.9 1) (layers "B.Cu" "B.Paste" "B.Mask") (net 11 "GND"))
  (pad "2" smd rect (at 1.65 6.35 270) (size 1.9 1) (layers "B.Cu" "B.Paste" "B.Mask") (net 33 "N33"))
  (pad "3" smd rect (at -1.65 3.81 270) (size 1.9 1) (layers "B.Cu" "B.Paste" "B.Mask") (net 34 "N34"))
  (pad "4" smd rect (at 1.65 1.27 270) (size 1.9 1) (layers "B.Cu" "B.Paste" "B.Mask") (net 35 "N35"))
  (pad "5" smd rect (at -1.65 -1.27 270) (size 1.9 1) (layers "B.Cu" "B.Paste" "B.Mask") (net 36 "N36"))
  (pad "6" smd rect (at 1.65 -3.81 270) (size 1.9 1) (layers "B.Cu" "B.Paste" "B.Mask") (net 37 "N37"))
  (pad "7" smd rect (at -1.65 -6.35 270) (size 1.9 1) (layers "B.Cu" "B.Paste" "B.Mask") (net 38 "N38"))
  (pad "8" smd rect (at 1.65 -8.89 270) (size 1.9 1) (layers "B.Cu" "B.Paste" "B.Mask") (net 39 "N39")))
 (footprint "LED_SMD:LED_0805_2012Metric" (layer "B.Cu") (at 145.275 93.325)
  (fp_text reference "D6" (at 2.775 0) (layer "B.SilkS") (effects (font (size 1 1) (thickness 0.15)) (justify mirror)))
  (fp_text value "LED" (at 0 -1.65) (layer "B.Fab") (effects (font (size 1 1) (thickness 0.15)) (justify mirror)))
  (pad "1" smd roundrect (at -0.9375 0) (size 0.975 1.4) (layers "B.Cu" "B.Paste" "B.Mask") (roundrect_rratio 0.25) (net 26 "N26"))
  (pad "2" smd roundrect (at 0.9375 0) (size 0.975 1.4) (layers "B.Cu" "B.Paste" "B.Mask") (roundrect_rratio 0.25) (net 27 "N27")))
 (gr_line (start 232.625 92.115) (end 232.625 122.094185) (stroke (width 0.05) (type default)) (layer "Edge.Cuts"))
 (gr_line (start 215.625 75.115) (end 73.875 75.115) (stroke (width 0.05) (type default)) (layer "Edge.Cuts"))
 (gr_line (start 215.625 139.094185) (end 73.895815 139.094185) (stroke (width 0.05) (type default)) (layer "Edge.Cuts"))
 (gr_circle (center 97.475 90.8) (end 99.975 90.8) (stroke (width 0.05) (type default)) (fill none) (layer "Edge.Cuts"))
 (gr_circle (center 193.175 106.75) (end 195.675 106.75) (stroke (width 0.05) (type default)) (fill none) (layer "Edge.Cuts"))
 (gr_circle (center 97.475 122.8) (end 99.975 122.8) (stroke (width 0.05) (type default)) (fill none) (layer "Edge.Cuts"))
 (gr_arc (start 232.625 122.094185) (mid 227.645821 134.11501) (end 215.625 139.094185) (stroke (width 0.05) (type default))
  (layer "Edge.Cuts"))
 (gr_arc (start 56.875 92.115) (mid 61.854185 80.094185) (end 73.875 75.115) (stroke (width 0.05) (type default)) (layer "Edge.Cuts"))
 (gr_circle (center 193.375 122.8) (end 195.875 122.8) (stroke (width 0.05) (type default)) (fill none) (layer "Edge.Cuts"))
 (gr_line (start 56.875 92.115) (end 56.895815 122.094185) (stroke (width 0.05) (type default)) (layer "Edge.Cuts"))
 (gr_circle (center 193.175 90.8) (end 195.675 90.8) (stroke (width 0.05) (type default)) (fill none) (layer "Edge.Cuts"))
 (gr_arc (start 215.625 75.115) (mid 227.645815 80.094185) (end 232.625 92.115) (stroke (width 0.05) (type default)) (layer "Edge.Cuts"))
 (gr_circle (center 97.5 106.725) (end 100 106.725) (stroke (width 0.05) (type default)) (fill none) (layer "Edge.Cuts"))
 (gr_rect (start 120.925 94.875) (end 169.525 118.675) (stroke (width 0.1) (type default)) (fill none) (layer "Edge.Cuts"))
 (gr_arc (start 73.895815 139.094185) (mid 61.875001 134.114999) (end 56.895815 122.094185) (stroke (width 0.05) (type default))
  (layer "Edge.Cuts"))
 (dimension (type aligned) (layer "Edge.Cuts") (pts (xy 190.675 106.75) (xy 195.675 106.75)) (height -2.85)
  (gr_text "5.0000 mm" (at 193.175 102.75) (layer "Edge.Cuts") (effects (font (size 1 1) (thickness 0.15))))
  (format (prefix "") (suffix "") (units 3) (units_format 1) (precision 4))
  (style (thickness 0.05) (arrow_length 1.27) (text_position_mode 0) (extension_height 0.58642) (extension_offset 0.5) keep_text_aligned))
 (segment (start 172.858668 109.858668) (end 207.418668 109.858668) (width 0.2) (layer "B.Cu") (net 11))
 (segment (start 207.46 86.125) (end 207.46 109.9) (width 0.2) (layer "B.Cu") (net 11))
 (segment (start 83.38 82.8) (end 83.38 128.005) (width 0.2) (layer "B.Cu") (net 11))
 (segment (start 144.3 134.2) (end 144.375 134.2) (width 0.2) (layer "B.Cu") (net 11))
 (segment (start 130.4 89.425) (end 125.825 84.85) (width 0.2) (layer "B.Cu") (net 11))
 (segment (start 130.4 91.5875) (end 130.4 89.425) (width 0.2) (layer "B.Cu") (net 11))
 (segment (start 204.69 134.2) (end 207.49 131.4) (width 0.2) (layer "B.Cu") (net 11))
 (segment (start 134.0125 120.25) (end 144.3375 120.25) (width 0.2) (layer "B.Cu") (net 11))
 (segment (start 171.075 107.6875) (end 171.075 108.075) (width 0.2) (layer "B.Cu") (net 11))
 (segment (start 171.075 108.075) (end 172.858668 109.858668) (width 0.2) (layer "B.Cu") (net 11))
 (segment (start 207.418668 109.858668) (end 207.46 109.9) (width 0.2) (layer "B.Cu") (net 11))
 (segment (start 85.43 84.85) (end 83.38 82.8) (width 0.2) (layer "B.Cu") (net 11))
 (segment (start 125.825 84.85) (end 85.43 84.85) (width 0.2) (layer "B.Cu") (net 11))
 (segment (start 84.8 134.2) (end 144.3 134.2) (width 0.2) (layer "B.Cu") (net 11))
 (segment (start 144.3375 120.25) (end 144.3375 134.1625) (width 0.2) (layer "B.Cu") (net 11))
 (segment (start 83.31 128.075) (end 83.31 132.71) (width 0.2) (layer "B.Cu") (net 11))
 (segment (start 83.38 128.005) (end 83.31 128.075) (width 0.2) (layer "B.Cu") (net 11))
 (segment (start 144.375 134.2) (end 204.69 134.2) (width 0.2) (layer "B.Cu") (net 11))
 (segment (start 144.3375 134.1625) (end 144.3 134.2) (width 0.2) (layer "B.Cu") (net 11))
 (segment (start 207.46 131.37) (end 207.49 131.4) (width 0.2) (layer "B.Cu") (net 11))
 (segment (start 83.31 132.71) (end 84.8 134.2) (width 0.2) (layer "B.Cu") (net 11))
 (segment (start 207.46 109.9) (end 207.46 131.37) (width 0.2) (layer "B.Cu") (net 11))
 (segment (start 132.1375 93.325) (end 130.4 91.5875) (width 0.2) (layer "B.Cu") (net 11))
 (segment (start 144.3125 93.3) (end 134.0375 93.3) (width 0.2) (layer "B.Cu") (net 26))
 (segment (start 134.0375 93.3) (end 134.0125 93.325) (width 0.2) (layer "B.Cu") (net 26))
 (segment (start 144.3375 93.325) (end 144.3125 93.3) (width 0.2) (layer "B.Cu") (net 26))
 (segment (start 181.225 88.65) (end 178.875 88.65) (width 0.2) (layer "B.Cu") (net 7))
 (segment (start 177.775 85.9) (end 180.85 82.825) (width 0.2) (layer "B.Cu") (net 7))
 (segment (start 180.85 82.825) (end 189.68 82.825) (width 0.2) (layer "B.Cu") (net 7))
 (segment (start 178.875 88.65) (end 177.775 87.55) (width 0.2) (layer "B.Cu") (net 7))
 (segment (start 177.775 87.55) (end 177.775 85.9) (width 0.2) (layer "B.Cu") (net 7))
 (segment (start 202.65 82.825) (end 197.775 87.7) (width 0.2) (layer "B.Cu") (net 9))
 (segment (start 204.92 82.825) (end 202.65 82.825) (width 0.2) (layer "B.Cu") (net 9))
 (segment (start 197.775 87.7) (end 183.1 87.7) (width 0.2) (layer "B.Cu") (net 9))
 (segment (start 119.375 105.8125) (end 119.35 105.7875) (width 0.2) (layer "B.Cu") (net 2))
 (segment (start 122.075 90.525) (end 129.4625 90.525) (width 0.2) (layer "B.Cu") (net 2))
 (segment (start 119.35 105.7875) (end 119.35 93.25) (width 0.2) (layer "B.Cu") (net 2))
 (segment (start 119.35 93.25) (end 122.075 90.525) (width 0.2) (layer "B.Cu") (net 2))
 (segment (start 146.2125 120.25) (end 156.4375 120.25) (width 0.2) (layer "B.Cu") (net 3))
 (segment (start 120.325 120.375) (end 119.375 119.425) (width 0.2) (layer "B.Cu") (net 1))
 (segment (start 132.0125 120.375) (end 120.325 120.375) (width 0.2) (layer "B.Cu") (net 1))
 (segment (start 132.1375 120.25) (end 132.0125 120.375) (width 0.2) (layer "B.Cu") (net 1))
 (segment (start 119.375 119.425) (end 119.375 107.6875) (width 0.2) (layer "B.Cu") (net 1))
 (segment (start 171.025 105.7625) (end 171.075 105.8125) (width 0.2) (layer "B.Cu") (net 5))
 (segment (start 158.3625 93.35) (end 169.9 93.35) (width 0.2) (layer "B.Cu") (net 5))
 (segment (start 158.3375 93.325) (end 158.3625 93.35) (width 0.2) (layer "B.Cu") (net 5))
 (segment (start 169.9 93.35) (end 171.025 94.475) (width 0.2) (layer "B.Cu") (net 5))
 (segment (start 171.025 94.475) (end 171.025 105.7625) (width 0.2) (layer "B.Cu") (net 5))
 (segment (start 181.225 86.75) (end 178.65 86.75) (width 0.2) (layer "B.Cu") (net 8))
 (segment (start 174.025 117.8) (end 174.025 110.8125) (width 0.2) (layer "B.Cu") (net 4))
 (segment (start 158.3125 120.25) (end 171.575 120.25) (width 0.2) (layer "B.Cu") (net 4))
 (segment (start 171.575 120.25) (end 174.025 117.8) (width 0.2) (layer "B.Cu") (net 4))
 (segment (start 146.2125 90.525) (end 146.2125 93.325) (width 0.2) (layer "B.Cu") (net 27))
 (segment (start 156.4375 93.725) (end 156.4625 93.75) (width 0.2) (layer "B.Cu") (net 6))
 (segment (start 156.4375 90.525) (end 156.4375 93.725) (width 0.2) (layer "B.Cu") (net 6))
 (segment (start 132.3375 89.525) (end 131.3375 90.525) (width 0.2) (layer "B.Cu") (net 10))
 (segment (start 148.0875 90.525) (end 147.0875 89.525) (width 0.2) (layer "B.Cu") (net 10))
 (segment (start 158.3125 90.525) (end 157.3125 89.525) (width 0.2) (layer "B.Cu") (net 10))
 (segment (start 158.3125 90.525) (end 162.0875 86.75) (width 0.2) (layer "B.Cu") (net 10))
 (segment (start 174.025 108.9375) (end 177 105.9625) (width 0.2) (layer "B.Cu") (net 10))
 (segment (start 147.0875 89.525) (end 132.3375 89.525) (width 0.2) (layer "B.Cu") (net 10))
 (segment (start 149.0875 89.525) (end 148.0875 90.525) (width 0.2) (layer "B.Cu") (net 10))
 (segment (start 157.3125 89.525) (end 149.0875 89.525) (width 0.2) (layer "B.Cu") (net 10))
 (segment (start 162.0875 86.75) (end 177 86.75) (width 0.2) (layer "B.Cu") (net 10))
 (segment (start 177 105.9625) (end 177 86.75) (width 0.2) (layer "B.Cu") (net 10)))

